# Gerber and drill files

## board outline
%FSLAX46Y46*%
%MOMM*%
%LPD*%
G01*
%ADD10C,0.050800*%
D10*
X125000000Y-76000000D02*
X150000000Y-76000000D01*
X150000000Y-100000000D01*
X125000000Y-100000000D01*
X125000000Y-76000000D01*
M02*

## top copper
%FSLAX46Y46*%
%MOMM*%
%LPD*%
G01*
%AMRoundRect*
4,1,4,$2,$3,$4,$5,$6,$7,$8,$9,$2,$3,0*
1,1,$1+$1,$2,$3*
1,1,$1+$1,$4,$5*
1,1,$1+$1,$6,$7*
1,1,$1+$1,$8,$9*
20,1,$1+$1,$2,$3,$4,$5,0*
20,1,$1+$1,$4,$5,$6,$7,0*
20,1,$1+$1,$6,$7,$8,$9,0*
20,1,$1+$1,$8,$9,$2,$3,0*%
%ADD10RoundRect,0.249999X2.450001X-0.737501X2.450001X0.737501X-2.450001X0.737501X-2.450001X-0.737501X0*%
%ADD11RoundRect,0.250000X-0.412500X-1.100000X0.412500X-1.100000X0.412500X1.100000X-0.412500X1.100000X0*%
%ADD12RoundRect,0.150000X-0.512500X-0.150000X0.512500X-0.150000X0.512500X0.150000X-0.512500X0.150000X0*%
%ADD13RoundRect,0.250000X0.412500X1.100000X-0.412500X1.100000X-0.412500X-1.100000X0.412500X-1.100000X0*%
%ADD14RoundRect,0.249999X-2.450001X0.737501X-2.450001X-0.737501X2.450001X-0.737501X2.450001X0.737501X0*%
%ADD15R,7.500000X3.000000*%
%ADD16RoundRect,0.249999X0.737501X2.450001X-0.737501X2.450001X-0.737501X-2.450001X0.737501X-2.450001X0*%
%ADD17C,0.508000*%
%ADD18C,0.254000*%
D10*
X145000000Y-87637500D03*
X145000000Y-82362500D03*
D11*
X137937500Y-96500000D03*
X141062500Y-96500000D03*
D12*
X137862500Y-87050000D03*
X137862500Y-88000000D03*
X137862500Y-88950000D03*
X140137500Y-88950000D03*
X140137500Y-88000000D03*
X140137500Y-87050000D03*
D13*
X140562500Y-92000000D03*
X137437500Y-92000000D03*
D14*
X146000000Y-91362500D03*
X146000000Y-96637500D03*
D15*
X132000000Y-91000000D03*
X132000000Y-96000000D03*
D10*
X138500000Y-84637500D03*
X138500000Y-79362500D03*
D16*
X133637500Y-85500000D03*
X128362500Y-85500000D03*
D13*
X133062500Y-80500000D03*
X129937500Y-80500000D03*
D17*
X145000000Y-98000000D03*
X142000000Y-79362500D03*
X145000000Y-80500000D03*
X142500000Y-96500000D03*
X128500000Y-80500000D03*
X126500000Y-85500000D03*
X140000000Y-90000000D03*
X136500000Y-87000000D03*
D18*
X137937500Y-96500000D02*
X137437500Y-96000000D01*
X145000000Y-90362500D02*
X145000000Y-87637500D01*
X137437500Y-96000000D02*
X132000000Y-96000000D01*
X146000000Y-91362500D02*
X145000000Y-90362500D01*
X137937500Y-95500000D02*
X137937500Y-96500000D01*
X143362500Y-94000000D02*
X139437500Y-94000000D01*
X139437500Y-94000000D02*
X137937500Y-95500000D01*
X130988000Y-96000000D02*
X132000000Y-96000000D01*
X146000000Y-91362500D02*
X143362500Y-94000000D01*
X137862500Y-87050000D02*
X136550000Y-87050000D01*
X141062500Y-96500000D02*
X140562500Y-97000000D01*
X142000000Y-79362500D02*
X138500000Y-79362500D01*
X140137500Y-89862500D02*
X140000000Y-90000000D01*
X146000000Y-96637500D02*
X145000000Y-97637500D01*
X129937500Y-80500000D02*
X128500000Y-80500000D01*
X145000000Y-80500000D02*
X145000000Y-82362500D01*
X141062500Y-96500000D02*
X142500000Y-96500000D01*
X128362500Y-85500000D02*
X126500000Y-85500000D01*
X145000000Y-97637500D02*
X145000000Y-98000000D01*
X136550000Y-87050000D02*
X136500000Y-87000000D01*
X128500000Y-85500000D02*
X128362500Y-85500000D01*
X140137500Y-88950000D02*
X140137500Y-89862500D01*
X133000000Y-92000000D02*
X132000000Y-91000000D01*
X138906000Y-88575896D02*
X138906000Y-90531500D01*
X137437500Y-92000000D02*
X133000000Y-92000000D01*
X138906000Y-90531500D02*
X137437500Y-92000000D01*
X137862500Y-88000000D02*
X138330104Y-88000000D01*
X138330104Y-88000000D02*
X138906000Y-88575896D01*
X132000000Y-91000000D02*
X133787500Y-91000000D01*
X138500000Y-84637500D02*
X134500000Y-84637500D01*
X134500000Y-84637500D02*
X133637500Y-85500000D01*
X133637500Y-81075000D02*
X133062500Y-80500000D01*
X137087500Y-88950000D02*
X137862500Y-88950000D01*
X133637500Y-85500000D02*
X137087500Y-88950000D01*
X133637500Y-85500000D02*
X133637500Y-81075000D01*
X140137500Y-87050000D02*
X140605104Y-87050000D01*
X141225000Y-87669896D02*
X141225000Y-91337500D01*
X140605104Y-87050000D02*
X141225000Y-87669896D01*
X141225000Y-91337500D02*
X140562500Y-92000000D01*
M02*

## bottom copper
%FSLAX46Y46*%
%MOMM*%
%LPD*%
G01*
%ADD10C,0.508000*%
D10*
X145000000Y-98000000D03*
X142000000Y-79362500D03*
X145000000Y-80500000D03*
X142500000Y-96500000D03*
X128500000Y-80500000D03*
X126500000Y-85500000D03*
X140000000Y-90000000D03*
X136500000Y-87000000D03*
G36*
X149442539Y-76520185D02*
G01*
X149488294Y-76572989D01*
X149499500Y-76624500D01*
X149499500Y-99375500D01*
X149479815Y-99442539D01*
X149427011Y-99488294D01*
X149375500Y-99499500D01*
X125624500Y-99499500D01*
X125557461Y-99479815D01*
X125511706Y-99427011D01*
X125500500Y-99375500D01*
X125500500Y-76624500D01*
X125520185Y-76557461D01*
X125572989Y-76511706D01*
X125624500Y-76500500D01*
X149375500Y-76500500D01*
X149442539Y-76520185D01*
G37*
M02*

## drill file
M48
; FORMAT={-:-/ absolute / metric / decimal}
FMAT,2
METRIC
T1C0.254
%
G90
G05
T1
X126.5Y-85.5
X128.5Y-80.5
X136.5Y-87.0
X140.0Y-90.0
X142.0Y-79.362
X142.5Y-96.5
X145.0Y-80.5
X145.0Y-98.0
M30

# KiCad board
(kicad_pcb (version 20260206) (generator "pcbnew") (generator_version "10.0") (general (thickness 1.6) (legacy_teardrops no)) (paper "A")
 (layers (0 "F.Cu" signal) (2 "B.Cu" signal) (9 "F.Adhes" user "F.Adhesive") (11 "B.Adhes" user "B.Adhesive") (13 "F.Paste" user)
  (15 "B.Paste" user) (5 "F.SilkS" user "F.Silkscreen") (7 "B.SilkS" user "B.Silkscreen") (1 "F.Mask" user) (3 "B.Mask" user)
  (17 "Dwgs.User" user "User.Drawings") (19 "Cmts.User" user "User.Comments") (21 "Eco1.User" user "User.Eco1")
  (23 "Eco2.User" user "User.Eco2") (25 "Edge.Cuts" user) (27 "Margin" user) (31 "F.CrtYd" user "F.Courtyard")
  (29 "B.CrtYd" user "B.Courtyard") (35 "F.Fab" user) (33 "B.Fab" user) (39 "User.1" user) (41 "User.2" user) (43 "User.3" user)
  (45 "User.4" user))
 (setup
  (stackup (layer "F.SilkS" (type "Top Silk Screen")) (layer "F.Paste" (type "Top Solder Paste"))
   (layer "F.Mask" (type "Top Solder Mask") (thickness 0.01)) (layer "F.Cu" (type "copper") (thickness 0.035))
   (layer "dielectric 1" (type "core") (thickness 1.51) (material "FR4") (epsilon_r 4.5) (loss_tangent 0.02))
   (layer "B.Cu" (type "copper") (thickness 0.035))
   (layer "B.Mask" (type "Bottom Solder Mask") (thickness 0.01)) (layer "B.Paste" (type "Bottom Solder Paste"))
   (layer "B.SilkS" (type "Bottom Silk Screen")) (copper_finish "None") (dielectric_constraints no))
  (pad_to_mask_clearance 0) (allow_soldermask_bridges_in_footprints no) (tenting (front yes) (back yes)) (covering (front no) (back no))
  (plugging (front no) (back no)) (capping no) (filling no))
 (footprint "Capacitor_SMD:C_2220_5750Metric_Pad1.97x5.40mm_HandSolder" (layer "F.Cu") (at 145 85 90)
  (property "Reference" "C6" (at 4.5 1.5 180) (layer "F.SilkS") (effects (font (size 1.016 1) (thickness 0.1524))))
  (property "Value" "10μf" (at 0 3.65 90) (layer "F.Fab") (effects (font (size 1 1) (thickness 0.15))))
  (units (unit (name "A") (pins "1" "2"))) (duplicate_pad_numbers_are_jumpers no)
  (pad "1" smd roundrect (at -2.6375 0 90) (size 1.975 5.4) (layers "F.Cu" "F.Mask" "F.Paste") (roundrect_rratio 0.126582) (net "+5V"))
  (pad "2" smd roundrect (at 2.6375 0 90) (size 1.975 5.4) (layers "F.Cu" "F.Mask" "F.Paste") (roundrect_rratio 0.126582) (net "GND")))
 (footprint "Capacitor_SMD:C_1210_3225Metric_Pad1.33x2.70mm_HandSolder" (layer "F.Cu") (at 139.5 96.5)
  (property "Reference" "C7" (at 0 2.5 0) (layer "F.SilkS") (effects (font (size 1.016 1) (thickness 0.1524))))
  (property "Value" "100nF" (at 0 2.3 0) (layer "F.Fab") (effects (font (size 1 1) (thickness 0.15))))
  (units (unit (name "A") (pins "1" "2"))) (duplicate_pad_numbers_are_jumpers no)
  (pad "1" smd roundrect (at -1.5625 0) (size 1.325 2.7) (layers "F.Cu" "F.Mask" "F.Paste") (roundrect_rratio 0.188679) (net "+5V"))
  (pad "2" smd roundrect (at 1.5625 0) (size 1.325 2.7) (layers "F.Cu" "F.Mask" "F.Paste") (roundrect_rratio 0.188679) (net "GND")))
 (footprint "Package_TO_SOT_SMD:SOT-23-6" (layer "F.Cu") (at 139 88)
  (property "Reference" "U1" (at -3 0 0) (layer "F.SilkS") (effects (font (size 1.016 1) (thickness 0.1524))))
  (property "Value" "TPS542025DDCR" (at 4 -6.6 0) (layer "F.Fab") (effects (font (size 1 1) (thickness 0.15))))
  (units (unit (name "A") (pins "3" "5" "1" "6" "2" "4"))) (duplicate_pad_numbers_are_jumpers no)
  (pad "1" smd roundrect (at -1.1375 -0.95) (size 1.325 0.6) (layers "F.Cu" "F.Mask" "F.Paste") (roundrect_rratio 0.25) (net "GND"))
  (pad "2" smd roundrect (at -1.1375 0) (size 1.325 0.6) (layers "F.Cu" "F.Mask" "F.Paste") (roundrect_rratio 0.25) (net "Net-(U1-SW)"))
  (pad "3" smd roundrect (at -1.1375 0.95) (size 1.325 0.6) (layers "F.Cu" "F.Mask" "F.Paste") (roundrect_rratio 0.25) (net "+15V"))
  (pad "4" smd roundrect (at 1.1375 0.95) (size 1.325 0.6) (layers "F.Cu" "F.Mask" "F.Paste") (roundrect_rratio 0.25) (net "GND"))
  (pad "5" smd roundrect (at 1.1375 0) (size 1.325 0.6) (layers "F.Cu" "F.Mask" "F.Paste") (roundrect_rratio 0.25)
   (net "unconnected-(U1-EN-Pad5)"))
  (pad "6" smd roundrect (at 1.1375 -0.95) (size 1.325 0.6) (layers "F.Cu" "F.Mask" "F.Paste") (roundrect_rratio 0.25) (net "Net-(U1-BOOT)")))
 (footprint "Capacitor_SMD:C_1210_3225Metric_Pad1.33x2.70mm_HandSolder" (layer "F.Cu") (at 139 92 180)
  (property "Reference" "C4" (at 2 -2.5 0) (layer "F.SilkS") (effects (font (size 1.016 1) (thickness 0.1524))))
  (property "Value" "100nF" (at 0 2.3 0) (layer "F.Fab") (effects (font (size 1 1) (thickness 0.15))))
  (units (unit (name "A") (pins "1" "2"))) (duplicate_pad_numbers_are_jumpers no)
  (pad "1" smd roundrect (at -1.5625 0 180) (size 1.325 2.7) (layers "F.Cu" "F.Mask" "F.Paste") (roundrect_rratio 0.188679)
   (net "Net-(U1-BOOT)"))
  (pad "2" smd roundrect (at 1.5625 0 180) (size 1.325 2.7) (layers "F.Cu" "F.Mask" "F.Paste") (roundrect_rratio 0.188679)
   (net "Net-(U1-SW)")))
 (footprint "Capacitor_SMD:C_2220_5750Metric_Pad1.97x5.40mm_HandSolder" (layer "F.Cu") (at 146 94 -90)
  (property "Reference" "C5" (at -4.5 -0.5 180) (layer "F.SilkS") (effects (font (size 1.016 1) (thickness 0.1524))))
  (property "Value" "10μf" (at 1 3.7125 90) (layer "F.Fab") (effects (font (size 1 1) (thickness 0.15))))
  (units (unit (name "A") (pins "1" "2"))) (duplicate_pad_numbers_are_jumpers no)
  (pad "1" smd roundrect (at -2.6375 0 270) (size 1.975 5.4) (layers "F.Cu" "F.Mask" "F.Paste") (roundrect_rratio 0.126582) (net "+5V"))
  (pad "2" smd roundrect (at 2.6375 0 270) (size 1.975 5.4) (layers "F.Cu" "F.Mask" "F.Paste") (roundrect_rratio 0.126582) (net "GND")))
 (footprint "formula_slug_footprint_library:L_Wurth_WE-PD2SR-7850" (layer "F.Cu") (at 132 93.5 -90)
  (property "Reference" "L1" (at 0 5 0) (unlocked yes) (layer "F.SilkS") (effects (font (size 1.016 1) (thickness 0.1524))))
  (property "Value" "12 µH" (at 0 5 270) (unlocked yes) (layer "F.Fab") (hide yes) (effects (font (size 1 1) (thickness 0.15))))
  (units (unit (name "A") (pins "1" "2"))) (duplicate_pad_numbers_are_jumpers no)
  (pad "1" smd rect (at -2.5 0 270) (size 3 7.5) (layers "F.Cu" "F.Mask" "F.Paste") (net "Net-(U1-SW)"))
  (pad "2" smd rect (at 2.5 0 270) (size 3 7.5) (layers "F.Cu" "F.Mask" "F.Paste") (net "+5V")))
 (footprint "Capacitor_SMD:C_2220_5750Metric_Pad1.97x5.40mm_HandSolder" (layer "F.Cu") (at 138.5 82 90)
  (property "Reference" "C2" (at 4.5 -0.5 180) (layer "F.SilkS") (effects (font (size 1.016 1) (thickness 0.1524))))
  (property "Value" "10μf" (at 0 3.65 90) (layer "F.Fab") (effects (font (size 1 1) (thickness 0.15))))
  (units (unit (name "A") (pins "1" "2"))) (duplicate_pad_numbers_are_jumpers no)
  (pad "1" smd roundrect (at -2.6375 0 90) (size 1.975 5.4) (layers "F.Cu" "F.Mask" "F.Paste") (roundrect_rratio 0.126582) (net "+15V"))
  (pad "2" smd roundrect (at 2.6375 0 90) (size 1.975 5.4) (layers "F.Cu" "F.Mask" "F.Paste") (roundrect_rratio 0.126582) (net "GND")))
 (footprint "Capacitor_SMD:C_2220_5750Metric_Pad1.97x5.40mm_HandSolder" (layer "F.Cu") (at 131 85.5 180)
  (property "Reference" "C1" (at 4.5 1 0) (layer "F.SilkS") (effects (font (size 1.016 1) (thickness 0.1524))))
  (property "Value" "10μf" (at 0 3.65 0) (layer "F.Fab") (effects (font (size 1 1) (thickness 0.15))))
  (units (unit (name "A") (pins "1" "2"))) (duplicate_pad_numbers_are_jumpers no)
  (pad "1" smd roundrect (at -2.6375 0 180) (size 1.975 5.4) (layers "F.Cu" "F.Mask" "F.Paste") (roundrect_rratio 0.126582) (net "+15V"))
  (pad "2" smd roundrect (at 2.6375 0 180) (size 1.975 5.4) (layers "F.Cu" "F.Mask" "F.Paste") (roundrect_rratio 0.126582) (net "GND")))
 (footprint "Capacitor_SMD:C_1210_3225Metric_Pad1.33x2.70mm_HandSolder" (layer "F.Cu") (at 131.5 80.5 180)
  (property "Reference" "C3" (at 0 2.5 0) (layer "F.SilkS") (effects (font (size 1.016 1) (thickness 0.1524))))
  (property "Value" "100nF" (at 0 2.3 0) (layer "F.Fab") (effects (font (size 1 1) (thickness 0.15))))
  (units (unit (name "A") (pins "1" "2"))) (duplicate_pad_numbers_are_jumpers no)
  (pad "1" smd roundrect (at -1.5625 0 180) (size 1.325 2.7) (layers "F.Cu" "F.Mask" "F.Paste") (roundrect_rratio 0.188679) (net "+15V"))
  (pad "2" smd roundrect (at 1.5625 0 180) (size 1.325 2.7) (layers "F.Cu" "F.Mask" "F.Paste") (roundrect_rratio 0.188679) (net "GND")))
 (gr_rect (start 125 76) (end 150 100) (stroke (width 0.0508) (type default)) (fill no) (layer "Edge.Cuts"))
 (segment (start 137.9375 96.5) (end 137.4375 96) (width 0.254) (layer "F.Cu") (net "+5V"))
 (segment (start 145 90.3625) (end 145 87.6375) (width 0.254) (layer "F.Cu") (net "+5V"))
 (segment (start 137.4375 96) (end 132 96) (width 0.254) (layer "F.Cu") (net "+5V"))
 (segment (start 146 91.3625) (end 145 90.3625) (width 0.254) (layer "F.Cu") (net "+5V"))
 (segment (start 137.9375 95.5) (end 137.9375 96.5) (width 0.254) (layer "F.Cu") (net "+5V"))
 (segment (start 143.3625 94) (end 139.4375 94) (width 0.254) (layer "F.Cu") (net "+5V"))
 (segment (start 139.4375 94) (end 137.9375 95.5) (width 0.254) (layer "F.Cu") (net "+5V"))
 (segment (start 130.988 96) (end 132 96) (width 0.254) (layer "F.Cu") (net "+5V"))
 (segment (start 146 91.3625) (end 143.3625 94) (width 0.254) (layer "F.Cu") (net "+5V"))
 (segment (start 137.8625 87.05) (end 136.55 87.05) (width 0.254) (layer "F.Cu") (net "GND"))
 (segment (start 141.0625 96.5) (end 140.5625 97) (width 0.254) (layer "F.Cu") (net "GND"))
 (segment (start 142 79.3625) (end 138.5 79.3625) (width 0.254) (layer "F.Cu") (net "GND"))
 (segment (start 140.1375 89.8625) (end 140 90) (width 0.254) (layer "F.Cu") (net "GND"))
 (segment (start 146 96.6375) (end 145 97.6375) (width 0.254) (layer "F.Cu") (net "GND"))
 (segment (start 129.9375 80.5) (end 128.5 80.5) (width 0.254) (layer "F.Cu") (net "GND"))
 (segment (start 145 80.5) (end 145 82.3625) (width 0.254) (layer "F.Cu") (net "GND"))
 (segment (start 141.0625 96.5) (end 142.5 96.5) (width 0.254) (layer "F.Cu") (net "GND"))
 (segment (start 128.3625 85.5) (end 126.5 85.5) (width 0.254) (layer "F.Cu") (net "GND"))
 (segment (start 145 97.6375) (end 145 98) (width 0.254) (layer "F.Cu") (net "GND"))
 (segment (start 136.55 87.05) (end 136.5 87) (width 0.254) (layer "F.Cu") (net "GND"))
 (segment (start 128.5 85.5) (end 128.3625 85.5) (width 0.254) (layer "F.Cu") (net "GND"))
 (segment (start 140.1375 88.95) (end 140.1375 89.8625) (width 0.254) (layer "F.Cu") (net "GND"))
 (via (at 145 98) (size 0.508) (drill 0.254) (layers "F.Cu" "B.Cu") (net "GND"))
 (via (at 142 79.3625) (size 0.508) (drill 0.254) (layers "F.Cu" "B.Cu") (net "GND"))
 (via (at 145 80.5) (size 0.508) (drill 0.254) (layers "F.Cu" "B.Cu") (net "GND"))
 (via (at 142.5 96.5) (size 0.508) (drill 0.254) (layers "F.Cu" "B.Cu") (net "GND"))
 (via (at 128.5 80.5) (size 0.508) (drill 0.254) (layers "F.Cu" "B.Cu") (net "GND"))
 (via (at 126.5 85.5) (size 0.508) (drill 0.254) (layers "F.Cu" "B.Cu") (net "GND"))
 (via (at 140 90) (size 0.508) (drill 0.254) (layers "F.Cu" "B.Cu") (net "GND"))
 (via (at 136.5 87) (size 0.508) (drill 0.254) (layers "F.Cu" "B.Cu") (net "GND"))
 (segment (start 133 92) (end 132 91) (width 0.254) (layer "F.Cu") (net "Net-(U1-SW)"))
 (segment (start 138.906 88.575896) (end 138.906 90.5315) (width 0.254) (layer "F.Cu") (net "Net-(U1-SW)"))
 (segment (start 137.4375 92) (end 133 92) (width 0.254) (layer "F.Cu") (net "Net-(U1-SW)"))
 (segment (start 138.906 90.5315) (end 137.4375 92) (width 0.254) (layer "F.Cu") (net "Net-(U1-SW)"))
 (segment (start 137.8625 88) (end 138.330104 88) (width 0.254) (layer "F.Cu") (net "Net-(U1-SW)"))
 (segment (start 138.330104 88) (end 138.906 88.575896) (width 0.254) (layer "F.Cu") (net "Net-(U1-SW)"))
 (segment (start 132 91) (end 133.7875 91) (width 0.254) (layer "F.Cu") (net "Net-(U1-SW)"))
 (segment (start 138.5 84.6375) (end 134.5 84.6375) (width 0.254) (layer "F.Cu") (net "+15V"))
 (segment (start 134.5 84.6375) (end 133.6375 85.5) (width 0.254) (layer "F.Cu") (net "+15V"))
 (segment (start 133.6375 81.075) (end 133.0625 80.5) (width 0.254) (layer "F.Cu") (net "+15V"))
 (segment (start 137.0875 88.95) (end 137.8625 88.95) (width 0.254) (layer "F.Cu") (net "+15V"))
 (segment (start 133.6375 85.5) (end 137.0875 88.95) (width 0.254) (layer "F.Cu") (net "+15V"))
 (segment (start 133.6375 85.5) (end 133.6375 81.075) (width 0.254) (layer "F.Cu") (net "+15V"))
 (segment (start 140.1375 87.05) (end 140.605104 87.05) (width 0.254) (layer "F.Cu") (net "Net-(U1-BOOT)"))
 (segment (start 141.225 87.669896) (end 141.225 91.3375) (width 0.254) (layer "F.Cu") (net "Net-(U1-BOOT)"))
 (segment (start 140.605104 87.05) (end 141.225 87.669896) (width 0.254) (layer "F.Cu") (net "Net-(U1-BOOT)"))
 (segment (start 141.225 91.3375) (end 140.5625 92) (width 0.254) (layer "F.Cu") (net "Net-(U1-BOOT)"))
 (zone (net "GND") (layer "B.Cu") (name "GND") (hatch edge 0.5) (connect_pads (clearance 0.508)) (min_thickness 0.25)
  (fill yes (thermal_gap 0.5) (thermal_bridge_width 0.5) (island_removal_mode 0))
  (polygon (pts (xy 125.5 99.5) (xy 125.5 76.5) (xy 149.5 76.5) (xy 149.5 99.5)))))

